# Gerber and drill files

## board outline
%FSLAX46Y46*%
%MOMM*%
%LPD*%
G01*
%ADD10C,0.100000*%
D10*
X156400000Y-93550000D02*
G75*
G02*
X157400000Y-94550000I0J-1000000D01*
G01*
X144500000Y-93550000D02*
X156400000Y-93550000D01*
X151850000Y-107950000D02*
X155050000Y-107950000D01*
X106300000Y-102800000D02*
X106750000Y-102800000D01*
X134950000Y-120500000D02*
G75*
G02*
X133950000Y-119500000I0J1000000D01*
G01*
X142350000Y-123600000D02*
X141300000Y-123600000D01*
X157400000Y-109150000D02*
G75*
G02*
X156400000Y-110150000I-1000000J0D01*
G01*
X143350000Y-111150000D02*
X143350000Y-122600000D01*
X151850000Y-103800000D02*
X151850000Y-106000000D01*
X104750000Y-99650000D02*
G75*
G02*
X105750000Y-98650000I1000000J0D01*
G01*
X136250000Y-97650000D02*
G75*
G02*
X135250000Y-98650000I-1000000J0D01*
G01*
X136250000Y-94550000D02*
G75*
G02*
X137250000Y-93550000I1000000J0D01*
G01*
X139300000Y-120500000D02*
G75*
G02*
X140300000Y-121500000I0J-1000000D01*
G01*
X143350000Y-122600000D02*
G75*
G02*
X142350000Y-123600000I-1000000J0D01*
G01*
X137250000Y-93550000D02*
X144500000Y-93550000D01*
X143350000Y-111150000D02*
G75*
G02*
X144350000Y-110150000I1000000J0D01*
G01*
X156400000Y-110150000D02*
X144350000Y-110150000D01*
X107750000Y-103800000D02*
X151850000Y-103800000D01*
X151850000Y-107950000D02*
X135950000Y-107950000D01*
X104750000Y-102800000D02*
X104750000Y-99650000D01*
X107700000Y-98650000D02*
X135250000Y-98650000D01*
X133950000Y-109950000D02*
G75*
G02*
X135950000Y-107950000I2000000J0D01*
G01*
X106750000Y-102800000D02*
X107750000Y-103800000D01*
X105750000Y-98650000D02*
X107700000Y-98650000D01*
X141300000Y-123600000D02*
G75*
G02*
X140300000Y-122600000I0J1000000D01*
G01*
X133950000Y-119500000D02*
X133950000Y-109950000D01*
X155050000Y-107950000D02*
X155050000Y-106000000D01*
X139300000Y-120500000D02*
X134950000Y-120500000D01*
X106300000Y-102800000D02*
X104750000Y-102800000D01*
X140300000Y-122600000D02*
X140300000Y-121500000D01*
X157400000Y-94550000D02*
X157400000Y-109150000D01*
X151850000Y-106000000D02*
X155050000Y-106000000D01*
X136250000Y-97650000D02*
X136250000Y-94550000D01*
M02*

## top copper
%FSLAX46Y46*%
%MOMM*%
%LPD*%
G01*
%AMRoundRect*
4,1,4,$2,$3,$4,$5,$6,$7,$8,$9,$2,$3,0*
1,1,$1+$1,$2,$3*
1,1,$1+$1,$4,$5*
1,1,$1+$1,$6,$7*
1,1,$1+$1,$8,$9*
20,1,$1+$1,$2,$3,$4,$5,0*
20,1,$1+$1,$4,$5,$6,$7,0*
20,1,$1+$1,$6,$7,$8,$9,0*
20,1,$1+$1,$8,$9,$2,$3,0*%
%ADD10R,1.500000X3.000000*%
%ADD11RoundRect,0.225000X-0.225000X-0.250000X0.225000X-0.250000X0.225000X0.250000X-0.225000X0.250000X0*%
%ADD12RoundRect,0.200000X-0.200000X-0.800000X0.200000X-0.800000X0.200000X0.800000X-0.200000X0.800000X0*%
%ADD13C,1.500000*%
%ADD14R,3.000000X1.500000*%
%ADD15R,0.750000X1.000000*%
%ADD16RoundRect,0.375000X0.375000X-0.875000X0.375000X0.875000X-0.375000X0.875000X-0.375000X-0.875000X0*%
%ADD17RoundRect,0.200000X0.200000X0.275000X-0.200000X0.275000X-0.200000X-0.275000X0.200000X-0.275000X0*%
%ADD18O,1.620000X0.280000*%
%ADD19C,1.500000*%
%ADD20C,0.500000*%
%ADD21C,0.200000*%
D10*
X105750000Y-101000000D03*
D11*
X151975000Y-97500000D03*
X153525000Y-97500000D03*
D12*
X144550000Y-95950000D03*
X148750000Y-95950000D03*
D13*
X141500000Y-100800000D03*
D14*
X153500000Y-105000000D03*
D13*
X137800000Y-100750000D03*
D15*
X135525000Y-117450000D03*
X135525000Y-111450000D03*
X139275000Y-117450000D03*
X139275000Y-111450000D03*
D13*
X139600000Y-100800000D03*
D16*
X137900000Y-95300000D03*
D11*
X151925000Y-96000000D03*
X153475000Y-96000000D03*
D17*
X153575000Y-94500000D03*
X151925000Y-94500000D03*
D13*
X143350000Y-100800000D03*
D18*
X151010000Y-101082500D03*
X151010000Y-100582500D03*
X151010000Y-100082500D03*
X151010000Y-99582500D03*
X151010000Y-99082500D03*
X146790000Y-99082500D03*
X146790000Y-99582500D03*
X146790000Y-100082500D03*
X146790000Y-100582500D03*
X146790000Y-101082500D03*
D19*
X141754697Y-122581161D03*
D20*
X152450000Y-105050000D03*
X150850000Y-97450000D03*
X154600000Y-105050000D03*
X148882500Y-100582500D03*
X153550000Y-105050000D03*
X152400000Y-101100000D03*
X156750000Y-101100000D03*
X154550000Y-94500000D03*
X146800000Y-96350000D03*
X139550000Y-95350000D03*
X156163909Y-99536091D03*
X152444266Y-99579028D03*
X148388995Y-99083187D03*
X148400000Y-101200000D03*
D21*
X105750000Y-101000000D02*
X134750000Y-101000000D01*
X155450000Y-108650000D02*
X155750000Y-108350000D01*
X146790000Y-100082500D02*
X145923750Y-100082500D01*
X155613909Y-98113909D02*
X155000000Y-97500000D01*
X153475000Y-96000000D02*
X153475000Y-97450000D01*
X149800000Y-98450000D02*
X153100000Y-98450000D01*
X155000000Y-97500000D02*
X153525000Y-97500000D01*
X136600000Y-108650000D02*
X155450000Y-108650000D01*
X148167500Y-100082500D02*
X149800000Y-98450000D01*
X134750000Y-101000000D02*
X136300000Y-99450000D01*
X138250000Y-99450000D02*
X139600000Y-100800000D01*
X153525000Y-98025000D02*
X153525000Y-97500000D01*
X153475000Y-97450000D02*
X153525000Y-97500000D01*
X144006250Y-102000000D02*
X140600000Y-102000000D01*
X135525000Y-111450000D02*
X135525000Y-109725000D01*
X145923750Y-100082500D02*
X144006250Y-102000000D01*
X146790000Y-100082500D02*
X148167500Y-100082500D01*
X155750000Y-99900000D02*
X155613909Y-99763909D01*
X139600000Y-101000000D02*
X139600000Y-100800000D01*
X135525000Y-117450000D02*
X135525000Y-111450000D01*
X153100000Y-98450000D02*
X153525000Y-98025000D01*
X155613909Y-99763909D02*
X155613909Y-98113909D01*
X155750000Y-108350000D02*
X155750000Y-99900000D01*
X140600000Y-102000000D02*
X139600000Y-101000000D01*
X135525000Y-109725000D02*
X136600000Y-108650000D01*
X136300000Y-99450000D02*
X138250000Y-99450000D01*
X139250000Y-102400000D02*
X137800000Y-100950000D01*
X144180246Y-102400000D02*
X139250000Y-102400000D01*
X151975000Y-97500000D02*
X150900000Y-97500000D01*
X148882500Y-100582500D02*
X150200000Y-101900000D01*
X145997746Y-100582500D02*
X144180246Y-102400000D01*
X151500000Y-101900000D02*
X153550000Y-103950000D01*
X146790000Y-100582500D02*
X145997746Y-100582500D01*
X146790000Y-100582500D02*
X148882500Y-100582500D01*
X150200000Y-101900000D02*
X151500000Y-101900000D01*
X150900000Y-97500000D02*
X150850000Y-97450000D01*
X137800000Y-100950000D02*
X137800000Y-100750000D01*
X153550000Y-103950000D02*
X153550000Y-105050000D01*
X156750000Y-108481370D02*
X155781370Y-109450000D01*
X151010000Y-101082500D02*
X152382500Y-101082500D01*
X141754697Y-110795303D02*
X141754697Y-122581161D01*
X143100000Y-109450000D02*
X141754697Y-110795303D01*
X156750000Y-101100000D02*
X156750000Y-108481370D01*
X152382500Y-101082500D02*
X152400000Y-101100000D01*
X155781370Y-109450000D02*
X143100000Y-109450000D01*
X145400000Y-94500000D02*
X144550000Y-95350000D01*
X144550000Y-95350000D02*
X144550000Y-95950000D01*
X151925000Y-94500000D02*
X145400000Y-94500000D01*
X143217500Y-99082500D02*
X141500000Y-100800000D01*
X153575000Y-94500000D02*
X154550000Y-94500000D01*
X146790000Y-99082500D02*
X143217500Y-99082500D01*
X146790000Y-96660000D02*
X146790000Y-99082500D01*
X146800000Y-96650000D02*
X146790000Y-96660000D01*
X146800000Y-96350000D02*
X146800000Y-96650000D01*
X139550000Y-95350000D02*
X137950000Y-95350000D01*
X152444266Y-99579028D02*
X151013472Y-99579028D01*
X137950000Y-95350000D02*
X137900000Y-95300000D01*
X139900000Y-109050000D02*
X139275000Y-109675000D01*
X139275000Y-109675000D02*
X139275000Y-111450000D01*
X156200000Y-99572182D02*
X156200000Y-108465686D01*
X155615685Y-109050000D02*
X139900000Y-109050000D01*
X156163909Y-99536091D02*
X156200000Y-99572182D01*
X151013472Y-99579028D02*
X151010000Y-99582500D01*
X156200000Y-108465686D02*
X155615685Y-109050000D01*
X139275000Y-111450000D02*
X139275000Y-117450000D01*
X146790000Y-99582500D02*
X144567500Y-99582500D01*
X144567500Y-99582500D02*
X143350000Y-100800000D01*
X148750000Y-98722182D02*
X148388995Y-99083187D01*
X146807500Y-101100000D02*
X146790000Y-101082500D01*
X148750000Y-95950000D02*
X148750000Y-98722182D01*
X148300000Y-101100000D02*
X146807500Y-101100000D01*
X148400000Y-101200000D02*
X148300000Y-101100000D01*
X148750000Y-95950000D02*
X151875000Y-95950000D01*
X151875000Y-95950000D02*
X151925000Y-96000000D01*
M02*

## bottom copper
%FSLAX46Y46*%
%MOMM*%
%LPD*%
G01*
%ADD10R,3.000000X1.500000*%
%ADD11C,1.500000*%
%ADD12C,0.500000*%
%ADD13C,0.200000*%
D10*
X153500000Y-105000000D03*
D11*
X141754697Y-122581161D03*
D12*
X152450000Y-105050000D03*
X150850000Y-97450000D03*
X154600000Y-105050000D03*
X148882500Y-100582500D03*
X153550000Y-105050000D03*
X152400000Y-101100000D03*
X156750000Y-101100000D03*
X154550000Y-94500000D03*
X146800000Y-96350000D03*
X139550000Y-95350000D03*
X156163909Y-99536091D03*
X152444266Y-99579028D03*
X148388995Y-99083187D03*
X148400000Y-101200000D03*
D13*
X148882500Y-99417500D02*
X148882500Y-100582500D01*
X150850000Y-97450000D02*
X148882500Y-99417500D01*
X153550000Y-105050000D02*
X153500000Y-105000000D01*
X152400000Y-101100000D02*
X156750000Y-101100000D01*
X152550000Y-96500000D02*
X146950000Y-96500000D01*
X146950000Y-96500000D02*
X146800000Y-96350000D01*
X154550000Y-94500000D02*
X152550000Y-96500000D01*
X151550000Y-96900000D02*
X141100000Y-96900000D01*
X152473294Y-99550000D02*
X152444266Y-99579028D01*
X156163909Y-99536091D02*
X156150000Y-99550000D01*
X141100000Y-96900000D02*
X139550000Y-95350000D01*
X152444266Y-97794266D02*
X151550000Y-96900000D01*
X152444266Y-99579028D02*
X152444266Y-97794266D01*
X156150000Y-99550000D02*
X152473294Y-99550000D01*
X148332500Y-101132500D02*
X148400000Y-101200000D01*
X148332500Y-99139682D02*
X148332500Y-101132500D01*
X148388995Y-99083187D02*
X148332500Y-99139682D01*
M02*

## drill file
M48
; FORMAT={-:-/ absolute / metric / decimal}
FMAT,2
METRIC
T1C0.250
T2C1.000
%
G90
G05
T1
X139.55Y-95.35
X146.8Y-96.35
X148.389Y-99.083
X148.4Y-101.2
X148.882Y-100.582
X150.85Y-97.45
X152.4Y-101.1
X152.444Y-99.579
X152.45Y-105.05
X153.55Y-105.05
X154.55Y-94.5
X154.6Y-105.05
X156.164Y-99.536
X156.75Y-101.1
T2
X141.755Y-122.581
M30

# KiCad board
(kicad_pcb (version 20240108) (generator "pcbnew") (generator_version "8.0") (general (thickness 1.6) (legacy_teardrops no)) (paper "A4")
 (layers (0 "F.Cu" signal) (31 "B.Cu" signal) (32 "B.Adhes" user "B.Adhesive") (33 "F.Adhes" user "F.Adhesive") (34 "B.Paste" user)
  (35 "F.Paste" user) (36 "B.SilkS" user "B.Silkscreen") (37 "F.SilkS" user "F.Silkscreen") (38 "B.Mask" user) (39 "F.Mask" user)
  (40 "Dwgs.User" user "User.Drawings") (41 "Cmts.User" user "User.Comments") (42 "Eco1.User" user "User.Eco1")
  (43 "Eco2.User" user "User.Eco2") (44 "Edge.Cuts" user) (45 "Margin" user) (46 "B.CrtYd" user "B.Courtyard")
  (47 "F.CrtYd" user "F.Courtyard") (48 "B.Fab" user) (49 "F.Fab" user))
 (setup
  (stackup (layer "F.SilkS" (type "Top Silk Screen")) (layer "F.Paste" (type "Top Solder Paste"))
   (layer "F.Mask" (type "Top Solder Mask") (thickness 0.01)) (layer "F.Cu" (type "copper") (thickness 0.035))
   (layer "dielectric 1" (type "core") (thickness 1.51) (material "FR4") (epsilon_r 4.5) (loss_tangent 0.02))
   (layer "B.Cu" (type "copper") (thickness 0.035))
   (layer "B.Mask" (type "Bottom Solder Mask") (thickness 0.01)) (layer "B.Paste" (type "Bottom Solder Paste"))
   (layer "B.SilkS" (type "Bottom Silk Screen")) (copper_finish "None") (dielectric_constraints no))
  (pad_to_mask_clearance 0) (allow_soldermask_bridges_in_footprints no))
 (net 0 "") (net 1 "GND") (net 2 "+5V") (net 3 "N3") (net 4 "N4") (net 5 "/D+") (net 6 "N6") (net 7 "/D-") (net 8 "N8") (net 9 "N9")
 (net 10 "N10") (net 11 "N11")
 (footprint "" (layer "F.Cu") (at 105.75 101 90)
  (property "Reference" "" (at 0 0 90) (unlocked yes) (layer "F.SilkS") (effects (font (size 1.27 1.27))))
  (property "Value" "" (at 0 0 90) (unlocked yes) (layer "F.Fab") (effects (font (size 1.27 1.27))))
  (pad "1" smd rect (at 0 0 90) (size 3 1.5) (layers "F.Cu" "F.Paste" "F.Mask") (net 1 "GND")))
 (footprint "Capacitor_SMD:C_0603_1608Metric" (layer "F.Cu") (at 152.75 97.5)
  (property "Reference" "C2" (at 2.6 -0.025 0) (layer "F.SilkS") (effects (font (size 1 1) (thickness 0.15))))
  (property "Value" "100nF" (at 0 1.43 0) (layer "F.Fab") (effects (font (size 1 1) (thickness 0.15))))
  (pad "1" smd roundrect (at -0.775 0) (size 0.9 0.95) (layers "F.Cu" "F.Paste" "F.Mask") (roundrect_rratio 0.25) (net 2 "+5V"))
  (pad "2" smd roundrect (at 0.775 0) (size 0.9 0.95) (layers "F.Cu" "F.Paste" "F.Mask") (roundrect_rratio 0.25) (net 1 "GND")))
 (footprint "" (layer "F.Cu") (at 153.5 105)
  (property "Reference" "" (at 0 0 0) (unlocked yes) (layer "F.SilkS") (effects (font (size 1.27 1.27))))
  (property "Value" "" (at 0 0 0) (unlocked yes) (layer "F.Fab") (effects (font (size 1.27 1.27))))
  (pad "1" smd rect (at 0 0) (size 3 1.5) (layers "B.Cu" "B.Paste" "B.Mask") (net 2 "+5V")))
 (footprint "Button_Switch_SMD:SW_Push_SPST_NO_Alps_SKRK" (layer "F.Cu") (at 146.65 95.95)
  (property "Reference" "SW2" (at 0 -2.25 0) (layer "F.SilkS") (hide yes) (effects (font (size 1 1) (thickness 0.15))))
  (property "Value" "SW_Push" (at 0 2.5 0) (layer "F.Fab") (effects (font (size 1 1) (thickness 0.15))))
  (pad "1" smd roundrect (at -2.1 0) (size 0.8 2) (layers "F.Cu" "F.Paste" "F.Mask") (roundrect_rratio 0.25) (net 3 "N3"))
  (pad "2" smd roundrect (at 2.1 0) (size 0.8 2) (layers "F.Cu" "F.Paste" "F.Mask") (roundrect_rratio 0.25) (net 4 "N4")))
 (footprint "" (layer "F.Cu") (at 141.5 100.8 180)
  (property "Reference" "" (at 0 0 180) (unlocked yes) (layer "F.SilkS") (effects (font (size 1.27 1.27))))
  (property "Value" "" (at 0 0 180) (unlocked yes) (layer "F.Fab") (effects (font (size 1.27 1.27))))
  (pad "1" smd circle (at 0 0 90) (size 1.5 1.5) (layers "F.Cu" "F.Paste" "F.Mask") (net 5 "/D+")))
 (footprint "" (layer "F.Cu") (at 153.5 105 90)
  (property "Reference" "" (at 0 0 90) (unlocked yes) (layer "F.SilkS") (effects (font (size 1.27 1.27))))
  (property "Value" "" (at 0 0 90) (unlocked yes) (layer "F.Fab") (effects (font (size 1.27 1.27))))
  (pad "1" smd rect (at 0 0) (size 3 1.5) (layers "F.Cu" "F.Paste" "F.Mask") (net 2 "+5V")))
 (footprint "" (layer "F.Cu") (at 137.8 100.75 180)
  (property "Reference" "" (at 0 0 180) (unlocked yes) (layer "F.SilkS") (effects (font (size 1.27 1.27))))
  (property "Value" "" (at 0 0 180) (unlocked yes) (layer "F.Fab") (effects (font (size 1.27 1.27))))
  (pad "1" smd circle (at 0 0 90) (size 1.5 1.5) (layers "F.Cu" "F.Paste" "F.Mask") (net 2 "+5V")))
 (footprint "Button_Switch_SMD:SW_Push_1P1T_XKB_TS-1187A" (layer "F.Cu") (at 137.4 114.45 90)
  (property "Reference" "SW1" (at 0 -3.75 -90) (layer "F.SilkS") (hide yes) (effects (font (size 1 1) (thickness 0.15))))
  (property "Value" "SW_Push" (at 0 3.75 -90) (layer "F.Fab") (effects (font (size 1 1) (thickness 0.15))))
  (pad "1" smd rect (at -3 -1.875 90) (size 1 0.75) (layers "F.Cu" "F.Paste" "F.Mask") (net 1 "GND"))
  (pad "1" smd rect (at 3 -1.875 90) (size 1 0.75) (layers "F.Cu" "F.Paste" "F.Mask") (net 1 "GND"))
  (pad "2" smd rect (at -3 1.875 90) (size 1 0.75) (layers "F.Cu" "F.Paste" "F.Mask") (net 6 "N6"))
  (pad "2" smd rect (at 3 1.875 90) (size 1 0.75) (layers "F.Cu" "F.Paste" "F.Mask") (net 6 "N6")))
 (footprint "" (layer "F.Cu") (at 139.6 100.8 180)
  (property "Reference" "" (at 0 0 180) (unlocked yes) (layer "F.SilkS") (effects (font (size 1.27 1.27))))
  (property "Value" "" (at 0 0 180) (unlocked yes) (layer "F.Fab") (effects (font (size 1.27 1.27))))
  (pad "1" smd circle (at 0 0 90) (size 1.5 1.5) (layers "F.Cu" "F.Paste" "F.Mask") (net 1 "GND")))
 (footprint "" (layer "F.Cu") (at 137.9 95.3)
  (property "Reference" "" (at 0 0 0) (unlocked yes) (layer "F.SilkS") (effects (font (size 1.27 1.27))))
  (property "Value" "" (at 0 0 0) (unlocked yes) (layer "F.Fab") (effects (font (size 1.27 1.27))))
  (pad "2" smd roundrect (at 0 0 90) (size 2.5 1.5) (layers "F.Cu" "F.Paste" "F.Mask") (roundrect_rratio 0.25) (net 6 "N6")))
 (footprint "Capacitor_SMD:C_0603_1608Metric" (layer "F.Cu") (at 152.7 96)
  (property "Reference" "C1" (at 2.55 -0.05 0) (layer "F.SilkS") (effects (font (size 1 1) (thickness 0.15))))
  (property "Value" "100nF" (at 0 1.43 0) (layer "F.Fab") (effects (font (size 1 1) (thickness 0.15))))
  (pad "1" smd roundrect (at -0.775 0) (size 0.9 0.95) (layers "F.Cu" "F.Paste" "F.Mask") (roundrect_rratio 0.25) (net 4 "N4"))
  (pad "2" smd roundrect (at 0.775 0) (size 0.9 0.95) (layers "F.Cu" "F.Paste" "F.Mask") (roundrect_rratio 0.25) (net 1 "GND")))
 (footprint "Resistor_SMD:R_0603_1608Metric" (layer "F.Cu") (at 152.75 94.5 180)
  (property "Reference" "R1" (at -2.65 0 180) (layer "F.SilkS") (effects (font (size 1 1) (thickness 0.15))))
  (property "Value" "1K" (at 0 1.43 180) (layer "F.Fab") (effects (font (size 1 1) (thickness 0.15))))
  (pad "1" smd roundrect (at -0.825 0 180) (size 0.8 0.95) (layers "F.Cu" "F.Paste" "F.Mask") (roundrect_rratio 0.25) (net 5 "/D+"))
  (pad "2" smd roundrect (at 0.825 0 180) (size 0.8 0.95) (layers "F.Cu" "F.Paste" "F.Mask") (roundrect_rratio 0.25) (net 3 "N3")))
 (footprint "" (layer "F.Cu") (at 143.35 100.8 180)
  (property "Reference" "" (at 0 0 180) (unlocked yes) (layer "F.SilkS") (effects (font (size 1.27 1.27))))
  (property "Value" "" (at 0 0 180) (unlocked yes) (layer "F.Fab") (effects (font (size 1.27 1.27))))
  (pad "1" smd circle (at 0 0 90) (size 1.5 1.5) (layers "F.Cu" "F.Paste" "F.Mask") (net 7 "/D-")))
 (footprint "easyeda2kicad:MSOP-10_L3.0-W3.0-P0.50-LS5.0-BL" (layer "F.Cu") (at 148.9 100.0825 90)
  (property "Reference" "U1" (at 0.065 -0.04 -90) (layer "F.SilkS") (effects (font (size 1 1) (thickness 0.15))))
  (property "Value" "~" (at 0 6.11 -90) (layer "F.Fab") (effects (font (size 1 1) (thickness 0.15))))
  (pad "1" smd oval (at -1 2.11 90) (size 0.28 1.62) (layers "F.Cu" "F.Paste" "F.Mask") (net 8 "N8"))
  (pad "2" smd oval (at -0.5 2.11 90) (size 0.28 1.62) (layers "F.Cu" "F.Paste" "F.Mask") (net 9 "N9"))
  (pad "3" smd oval (at 0 2.11 90) (size 0.28 1.62) (layers "F.Cu" "F.Paste" "F.Mask") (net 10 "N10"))
  (pad "4" smd oval (at 0.5 2.11 90) (size 0.28 1.62) (layers "F.Cu" "F.Paste" "F.Mask") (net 6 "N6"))
  (pad "5" smd oval (at 1 2.11 90) (size 0.28 1.62) (layers "F.Cu" "F.Paste" "F.Mask") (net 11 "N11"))
  (pad "6" smd oval (at 1 -2.11 90) (size 0.28 1.62) (layers "F.Cu" "F.Paste" "F.Mask") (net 5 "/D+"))
  (pad "7" smd oval (at 0.5 -2.11 90) (size 0.28 1.62) (layers "F.Cu" "F.Paste" "F.Mask") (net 7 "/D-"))
  (pad "8" smd oval (at 0 -2.11 90) (size 0.28 1.62) (layers "F.Cu" "F.Paste" "F.Mask") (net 1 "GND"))
  (pad "9" smd oval (at -0.5 -2.11 90) (size 0.28 1.62) (layers "F.Cu" "F.Paste" "F.Mask") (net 2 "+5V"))
  (pad "10" smd oval (at -1 -2.11 90) (size 0.28 1.62) (layers "F.Cu" "F.Paste" "F.Mask") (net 4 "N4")))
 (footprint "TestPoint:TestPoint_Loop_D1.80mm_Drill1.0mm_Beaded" (layer "F.Cu") (at 141.754697 122.581161)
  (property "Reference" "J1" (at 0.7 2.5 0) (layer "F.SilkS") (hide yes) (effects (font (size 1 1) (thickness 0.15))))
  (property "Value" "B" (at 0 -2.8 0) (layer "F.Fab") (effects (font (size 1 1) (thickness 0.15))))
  (pad "1" thru_hole circle (at 0 0) (size 1.5 1.5) (drill 1) (layers "*.Cu" "*.Mask") (remove_unused_layers no) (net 8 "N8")))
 (gr_arc (start 156.4 93.55) (mid 157.107107 93.842893) (end 157.4 94.55) (stroke (width 0.1) (type default)) (layer "Edge.Cuts"))
 (gr_line (start 144.5 93.55) (end 156.4 93.55) (stroke (width 0.1) (type default)) (layer "Edge.Cuts"))
 (gr_line (start 151.85 107.95) (end 155.05 107.95) (stroke (width 0.1) (type default)) (layer "Edge.Cuts"))
 (gr_line (start 106.3 102.8) (end 106.75 102.8) (stroke (width 0.1) (type default)) (layer "Edge.Cuts"))
 (gr_arc (start 134.95 120.5) (mid 134.242893 120.207107) (end 133.95 119.5) (stroke (width 0.1) (type default)) (layer "Edge.Cuts"))
 (gr_line (start 142.35 123.6) (end 141.3 123.6) (stroke (width 0.1) (type default)) (layer "Edge.Cuts"))
 (gr_arc (start 157.4 109.15) (mid 157.107107 109.857107) (end 156.4 110.15) (stroke (width 0.1) (type default)) (layer "Edge.Cuts"))
 (gr_line (start 143.35 111.15) (end 143.35 122.6) (stroke (width 0.1) (type default)) (layer "Edge.Cuts"))
 (gr_line (start 151.85 103.8) (end 151.85 106) (stroke (width 0.1) (type default)) (layer "Edge.Cuts"))
 (gr_arc (start 104.75 99.65) (mid 105.042893 98.942893) (end 105.75 98.65) (stroke (width 0.1) (type default)) (layer "Edge.Cuts"))
 (gr_arc (start 136.25 97.65) (mid 135.957107 98.357107) (end 135.25 98.65) (stroke (width 0.1) (type default)) (layer "Edge.Cuts"))
 (gr_arc (start 136.25 94.55) (mid 136.542893 93.842893) (end 137.25 93.55) (stroke (width 0.1) (type default)) (layer "Edge.Cuts"))
 (gr_arc (start 139.3 120.5) (mid 140.007107 120.792893) (end 140.3 121.5) (stroke (width 0.1) (type default)) (layer "Edge.Cuts"))
 (gr_arc (start 143.35 122.6) (mid 143.057107 123.307107) (end 142.35 123.6) (stroke (width 0.1) (type default)) (layer "Edge.Cuts"))
 (gr_line (start 137.25 93.55) (end 144.5 93.55) (stroke (width 0.1) (type default)) (layer "Edge.Cuts"))
 (gr_arc (start 143.35 111.15) (mid 143.642893 110.442893) (end 144.35 110.15) (stroke (width 0.1) (type default)) (layer "Edge.Cuts"))
 (gr_line (start 156.4 110.15) (end 144.35 110.15) (stroke (width 0.1) (type default)) (layer "Edge.Cuts"))
 (gr_line (start 107.75 103.8) (end 151.85 103.8) (stroke (width 0.1) (type default)) (layer "Edge.Cuts"))
 (gr_line (start 151.85 107.95) (end 135.95 107.95) (stroke (width 0.1) (type default)) (layer "Edge.Cuts"))
 (gr_line (start 104.75 102.8) (end 104.75 99.65) (stroke (width 0.1) (type default)) (layer "Edge.Cuts"))
 (gr_line (start 107.7 98.65) (end 135.25 98.65) (stroke (width 0.1) (type default)) (layer "Edge.Cuts"))
 (gr_arc (start 133.95 109.95) (mid 134.535786 108.535786) (end 135.95 107.95) (stroke (width 0.1) (type default)) (layer "Edge.Cuts"))
 (gr_line (start 106.75 102.8) (end 107.75 103.8) (stroke (width 0.1) (type default)) (layer "Edge.Cuts"))
 (gr_line (start 105.75 98.65) (end 107.7 98.65) (stroke (width 0.1) (type default)) (layer "Edge.Cuts"))
 (gr_arc (start 141.3 123.6) (mid 140.592893 123.307107) (end 140.3 122.6) (stroke (width 0.1) (type default)) (layer "Edge.Cuts"))
 (gr_line (start 133.95 119.5) (end 133.95 109.95) (stroke (width 0.1) (type default)) (layer "Edge.Cuts"))
 (gr_line (start 155.05 107.95) (end 155.05 106) (stroke (width 0.1) (type default)) (layer "Edge.Cuts"))
 (gr_line (start 139.3 120.5) (end 134.95 120.5) (stroke (width 0.1) (type default)) (layer "Edge.Cuts"))
 (gr_line (start 106.3 102.8) (end 104.75 102.8) (stroke (width 0.1) (type default)) (layer "Edge.Cuts"))
 (gr_line (start 140.3 122.6) (end 140.3 121.5) (stroke (width 0.1) (type default)) (layer "Edge.Cuts"))
 (gr_line (start 157.4 94.55) (end 157.4 109.15) (stroke (width 0.1) (type default)) (layer "Edge.Cuts"))
 (gr_line (start 151.85 106) (end 155.05 106) (stroke (width 0.1) (type default)) (layer "Edge.Cuts"))
 (gr_line (start 136.25 97.65) (end 136.25 94.55) (stroke (width 0.1) (type default)) (layer "Edge.Cuts"))
 (segment (start 105.75 101) (end 134.75 101) (width 0.2) (layer "F.Cu") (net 1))
 (segment (start 155.45 108.65) (end 155.75 108.35) (width 0.2) (layer "F.Cu") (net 1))
 (segment (start 146.79 100.0825) (end 145.92375 100.0825) (width 0.2) (layer "F.Cu") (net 1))
 (segment (start 155.613909 98.113909) (end 155 97.5) (width 0.2) (layer "F.Cu") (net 1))
 (segment (start 153.475 96) (end 153.475 97.45) (width 0.2) (layer "F.Cu") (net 1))
 (segment (start 149.8 98.45) (end 153.1 98.45) (width 0.2) (layer "F.Cu") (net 1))
 (segment (start 155 97.5) (end 153.525 97.5) (width 0.2) (layer "F.Cu") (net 1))
 (segment (start 136.6 108.65) (end 155.45 108.65) (width 0.2) (layer "F.Cu") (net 1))
 (segment (start 148.1675 100.0825) (end 149.8 98.45) (width 0.2) (layer "F.Cu") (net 1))
 (segment (start 134.75 101) (end 136.3 99.45) (width 0.2) (layer "F.Cu") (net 1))
 (segment (start 138.25 99.45) (end 139.6 100.8) (width 0.2) (layer "F.Cu") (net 1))
 (segment (start 153.525 98.025) (end 153.525 97.5) (width 0.2) (layer "F.Cu") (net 1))
 (segment (start 153.475 97.45) (end 153.525 97.5) (width 0.2) (layer "F.Cu") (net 1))
 (segment (start 144.00625 102) (end 140.6 102) (width 0.2) (layer "F.Cu") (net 1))
 (segment (start 135.525 111.45) (end 135.525 109.725) (width 0.2) (layer "F.Cu") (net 1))
 (segment (start 145.92375 100.0825) (end 144.00625 102) (width 0.2) (layer "F.Cu") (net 1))
 (segment (start 146.79 100.0825) (end 148.1675 100.0825) (width 0.2) (layer "F.Cu") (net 1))
 (segment (start 155.75 99.9) (end 155.613909 99.763909) (width 0.2) (layer "F.Cu") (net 1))
 (segment (start 139.6 101) (end 139.6 100.8) (width 0.2) (layer "F.Cu") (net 1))
 (segment (start 135.525 117.45) (end 135.525 111.45) (width 0.2) (layer "F.Cu") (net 1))
 (segment (start 153.1 98.45) (end 153.525 98.025) (width 0.2) (layer "F.Cu") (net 1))
 (segment (start 155.613909 99.763909) (end 155.613909 98.113909) (width 0.2) (layer "F.Cu") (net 1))
 (segment (start 155.75 108.35) (end 155.75 99.9) (width 0.2) (layer "F.Cu") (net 1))
 (segment (start 140.6 102) (end 139.6 101) (width 0.2) (layer "F.Cu") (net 1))
 (segment (start 135.525 109.725) (end 136.6 108.65) (width 0.2) (layer "F.Cu") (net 1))
 (segment (start 136.3 99.45) (end 138.25 99.45) (width 0.2) (layer "F.Cu") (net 1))
 (segment (start 139.25 102.4) (end 137.8 100.95) (width 0.2) (layer "F.Cu") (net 2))
 (segment (start 144.180246 102.4) (end 139.25 102.4) (width 0.2) (layer "F.Cu") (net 2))
 (segment (start 151.975 97.5) (end 150.9 97.5) (width 0.2) (layer "F.Cu") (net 2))
 (segment (start 148.8825 100.5825) (end 150.2 101.9) (width 0.2) (layer "F.Cu") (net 2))
 (segment (start 145.997746 100.5825) (end 144.180246 102.4) (width 0.2) (layer "F.Cu") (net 2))
 (segment (start 151.5 101.9) (end 153.55 103.95) (width 0.2) (layer "F.Cu") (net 2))
 (segment (start 146.79 100.5825) (end 145.997746 100.5825) (width 0.2) (layer "F.Cu") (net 2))
 (segment (start 146.79 100.5825) (end 148.8825 100.5825) (width 0.2) (layer "F.Cu") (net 2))
 (segment (start 150.2 101.9) (end 151.5 101.9) (width 0.2) (layer "F.Cu") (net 2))
 (segment (start 150.9 97.5) (end 150.85 97.45) (width 0.2) (layer "F.Cu") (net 2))
 (segment (start 137.8 100.95) (end 137.8 100.75) (width 0.2) (layer "F.Cu") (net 2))
 (segment (start 153.55 103.95) (end 153.55 105.05) (width 0.2) (layer "F.Cu") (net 2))
 (via (at 152.45 105.05) (size 0.5) (drill 0.25) (layers "F.Cu" "B.Cu") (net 2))
 (via (at 150.85 97.45) (size 0.5) (drill 0.25) (layers "F.Cu" "B.Cu") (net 2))
 (via (at 154.6 105.05) (size 0.5) (drill 0.25) (layers "F.Cu" "B.Cu") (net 2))
 (via (at 148.8825 100.5825) (size 0.5) (drill 0.25) (layers "F.Cu" "B.Cu") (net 2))
 (via (at 153.55 105.05) (size 0.5) (drill 0.25) (layers "F.Cu" "B.Cu") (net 2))
 (segment (start 148.8825 99.4175) (end 148.8825 100.5825) (width 0.2) (layer "B.Cu") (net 2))
 (segment (start 150.85 97.45) (end 148.8825 99.4175) (width 0.2) (layer "B.Cu") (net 2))
 (segment (start 153.55 105.05) (end 153.5 105) (width 0.2) (layer "B.Cu") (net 2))
 (segment (start 156.75 108.48137) (end 155.78137 109.45) (width 0.2) (layer "F.Cu") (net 8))
 (segment (start 151.01 101.0825) (end 152.3825 101.0825) (width 0.2) (layer "F.Cu") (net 8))
 (segment (start 141.754697 110.795303) (end 141.754697 122.581161) (width 0.2) (layer "F.Cu") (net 8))
 (segment (start 143.1 109.45) (end 141.754697 110.795303) (width 0.2) (layer "F.Cu") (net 8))
 (segment (start 156.75 101.1) (end 156.75 108.48137) (width 0.2) (layer "F.Cu") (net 8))
 (segment (start 152.3825 101.0825) (end 152.4 101.1) (width 0.2) (layer "F.Cu") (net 8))
 (segment (start 155.78137 109.45) (end 143.1 109.45) (width 0.2) (layer "F.Cu") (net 8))
 (via (at 152.4 101.1) (size 0.5) (drill 0.25) (layers "F.Cu" "B.Cu") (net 8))
 (via (at 156.75 101.1) (size 0.5) (drill 0.25) (layers "F.Cu" "B.Cu") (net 8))
 (segment (start 152.4 101.1) (end 156.75 101.1) (width 0.2) (layer "B.Cu") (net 8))
 (segment (start 145.4 94.5) (end 144.55 95.35) (width 0.2) (layer "F.Cu") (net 3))
 (segment (start 144.55 95.35) (end 144.55 95.95) (width 0.2) (layer "F.Cu") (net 3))
 (segment (start 151.925 94.5) (end 145.4 94.5) (width 0.2) (layer "F.Cu") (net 3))
 (segment (start 143.2175 99.0825) (end 141.5 100.8) (width 0.2) (layer "F.Cu") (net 5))
 (segment (start 153.575 94.5) (end 154.55 94.5) (width 0.2) (layer "F.Cu") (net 5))
 (segment (start 146.79 99.0825) (end 143.2175 99.0825) (width 0.2) (layer "F.Cu") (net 5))
 (segment (start 146.79 96.66) (end 146.79 99.0825) (width 0.2) (layer "F.Cu") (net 5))
 (segment (start 146.8 96.65) (end 146.79 96.66) (width 0.2) (layer "F.Cu") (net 5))
 (segment (start 146.8 96.35) (end 146.8 96.65) (width 0.2) (layer "F.Cu") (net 5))
 (via (at 154.55 94.5) (size 0.5) (drill 0.25) (layers "F.Cu" "B.Cu") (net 5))
 (via (at 146.8 96.35) (size 0.5) (drill 0.25) (layers "F.Cu" "B.Cu") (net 5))
 (segment (start 152.55 96.5) (end 146.95 96.5) (width 0.2) (layer "B.Cu") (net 5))
 (segment (start 146.95 96.5) (end 146.8 96.35) (width 0.2) (layer "B.Cu") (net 5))
 (segment (start 154.55 94.5) (end 152.55 96.5) (width 0.2) (layer "B.Cu") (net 5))
 (segment (start 139.55 95.35) (end 137.95 95.35) (width 0.2) (layer "F.Cu") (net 6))
 (segment (start 152.444266 99.579028) (end 151.013472 99.579028) (width 0.2) (layer "F.Cu") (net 6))
 (segment (start 137.95 95.35) (end 137.9 95.3) (width 0.2) (layer "F.Cu") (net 6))
 (segment (start 139.9 109.05) (end 139.275 109.675) (width 0.2) (layer "F.Cu") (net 6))
 (segment (start 139.275 109.675) (end 139.275 111.45) (width 0.2) (layer "F.Cu") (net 6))
 (segment (start 156.2 99.572182) (end 156.2 108.465686) (width 0.2) (layer "F.Cu") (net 6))
 (segment (start 155.615685 109.05) (end 139.9 109.05) (width 0.2) (layer "F.Cu") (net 6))
 (segment (start 156.163909 99.536091) (end 156.2 99.572182) (width 0.2) (layer "F.Cu") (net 6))
 (segment (start 151.013472 99.579028) (end 151.01 99.5825) (width 0.2) (layer "F.Cu") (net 6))
 (segment (start 156.2 108.465686) (end 155.615685 109.05) (width 0.2) (layer "F.Cu") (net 6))
 (segment (start 139.275 111.45) (end 139.275 117.45) (width 0.2) (layer "F.Cu") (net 6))
 (via (at 139.55 95.35) (size 0.5) (drill 0.25) (layers "F.Cu" "B.Cu") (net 6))
 (via (at 156.163909 99.536091) (size 0.5) (drill 0.25) (layers "F.Cu" "B.Cu") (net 6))
 (via (at 152.444266 99.579028) (size 0.5) (drill 0.25) (layers "F.Cu" "B.Cu") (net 6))
 (segment (start 151.55 96.9) (end 141.1 96.9) (width 0.2) (layer "B.Cu") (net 6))
 (segment (start 152.473294 99.55) (end 152.444266 99.579028) (width 0.2) (layer "B.Cu") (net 6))
 (segment (start 156.163909 99.536091) (end 156.15 99.55) (width 0.2) (layer "B.Cu") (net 6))
 (segment (start 141.1 96.9) (end 139.55 95.35) (width 0.2) (layer "B.Cu") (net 6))
 (segment (start 152.444266 97.794266) (end 151.55 96.9) (width 0.2) (layer "B.Cu") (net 6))
 (segment (start 152.444266 99.579028) (end 152.444266 97.794266) (width 0.2) (layer "B.Cu") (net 6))
 (segment (start 156.15 99.55) (end 152.473294 99.55) (width 0.2) (layer "B.Cu") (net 6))
 (segment (start 146.79 99.5825) (end 144.5675 99.5825) (width 0.2) (layer "F.Cu") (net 7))
 (segment (start 144.5675 99.5825) (end 143.35 100.8) (width 0.2) (layer "F.Cu") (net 7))
 (segment (start 148.75 98.722182) (end 148.388995 99.083187) (width 0.2) (layer "F.Cu") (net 4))
 (segment (start 146.8075 101.1) (end 146.79 101.0825) (width 0.2) (layer "F.Cu") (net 4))
 (segment (start 148.75 95.95) (end 148.75 98.722182) (width 0.2) (layer "F.Cu") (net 4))
 (segment (start 148.3 101.1) (end 146.8075 101.1) (width 0.2) (layer "F.Cu") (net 4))
 (segment (start 148.4 101.2) (end 148.3 101.1) (width 0.2) (layer "F.Cu") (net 4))
 (segment (start 148.75 95.95) (end 151.875 95.95) (width 0.2) (layer "F.Cu") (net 4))
 (segment (start 151.875 95.95) (end 151.925 96) (width 0.2) (layer "F.Cu") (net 4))
 (via (at 148.388995 99.083187) (size 0.5) (drill 0.25) (layers "F.Cu" "B.Cu") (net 4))
 (via (at 148.4 101.2) (size 0.5) (drill 0.25) (layers "F.Cu" "B.Cu") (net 4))
 (segment (start 148.3325 101.1325) (end 148.4 101.2) (width 0.2) (layer "B.Cu") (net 4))
 (segment (start 148.3325 99.139682) (end 148.3325 101.1325) (width 0.2) (layer "B.Cu") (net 4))
 (segment (start 148.388995 99.083187) (end 148.3325 99.139682) (width 0.2) (layer "B.Cu") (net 4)))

